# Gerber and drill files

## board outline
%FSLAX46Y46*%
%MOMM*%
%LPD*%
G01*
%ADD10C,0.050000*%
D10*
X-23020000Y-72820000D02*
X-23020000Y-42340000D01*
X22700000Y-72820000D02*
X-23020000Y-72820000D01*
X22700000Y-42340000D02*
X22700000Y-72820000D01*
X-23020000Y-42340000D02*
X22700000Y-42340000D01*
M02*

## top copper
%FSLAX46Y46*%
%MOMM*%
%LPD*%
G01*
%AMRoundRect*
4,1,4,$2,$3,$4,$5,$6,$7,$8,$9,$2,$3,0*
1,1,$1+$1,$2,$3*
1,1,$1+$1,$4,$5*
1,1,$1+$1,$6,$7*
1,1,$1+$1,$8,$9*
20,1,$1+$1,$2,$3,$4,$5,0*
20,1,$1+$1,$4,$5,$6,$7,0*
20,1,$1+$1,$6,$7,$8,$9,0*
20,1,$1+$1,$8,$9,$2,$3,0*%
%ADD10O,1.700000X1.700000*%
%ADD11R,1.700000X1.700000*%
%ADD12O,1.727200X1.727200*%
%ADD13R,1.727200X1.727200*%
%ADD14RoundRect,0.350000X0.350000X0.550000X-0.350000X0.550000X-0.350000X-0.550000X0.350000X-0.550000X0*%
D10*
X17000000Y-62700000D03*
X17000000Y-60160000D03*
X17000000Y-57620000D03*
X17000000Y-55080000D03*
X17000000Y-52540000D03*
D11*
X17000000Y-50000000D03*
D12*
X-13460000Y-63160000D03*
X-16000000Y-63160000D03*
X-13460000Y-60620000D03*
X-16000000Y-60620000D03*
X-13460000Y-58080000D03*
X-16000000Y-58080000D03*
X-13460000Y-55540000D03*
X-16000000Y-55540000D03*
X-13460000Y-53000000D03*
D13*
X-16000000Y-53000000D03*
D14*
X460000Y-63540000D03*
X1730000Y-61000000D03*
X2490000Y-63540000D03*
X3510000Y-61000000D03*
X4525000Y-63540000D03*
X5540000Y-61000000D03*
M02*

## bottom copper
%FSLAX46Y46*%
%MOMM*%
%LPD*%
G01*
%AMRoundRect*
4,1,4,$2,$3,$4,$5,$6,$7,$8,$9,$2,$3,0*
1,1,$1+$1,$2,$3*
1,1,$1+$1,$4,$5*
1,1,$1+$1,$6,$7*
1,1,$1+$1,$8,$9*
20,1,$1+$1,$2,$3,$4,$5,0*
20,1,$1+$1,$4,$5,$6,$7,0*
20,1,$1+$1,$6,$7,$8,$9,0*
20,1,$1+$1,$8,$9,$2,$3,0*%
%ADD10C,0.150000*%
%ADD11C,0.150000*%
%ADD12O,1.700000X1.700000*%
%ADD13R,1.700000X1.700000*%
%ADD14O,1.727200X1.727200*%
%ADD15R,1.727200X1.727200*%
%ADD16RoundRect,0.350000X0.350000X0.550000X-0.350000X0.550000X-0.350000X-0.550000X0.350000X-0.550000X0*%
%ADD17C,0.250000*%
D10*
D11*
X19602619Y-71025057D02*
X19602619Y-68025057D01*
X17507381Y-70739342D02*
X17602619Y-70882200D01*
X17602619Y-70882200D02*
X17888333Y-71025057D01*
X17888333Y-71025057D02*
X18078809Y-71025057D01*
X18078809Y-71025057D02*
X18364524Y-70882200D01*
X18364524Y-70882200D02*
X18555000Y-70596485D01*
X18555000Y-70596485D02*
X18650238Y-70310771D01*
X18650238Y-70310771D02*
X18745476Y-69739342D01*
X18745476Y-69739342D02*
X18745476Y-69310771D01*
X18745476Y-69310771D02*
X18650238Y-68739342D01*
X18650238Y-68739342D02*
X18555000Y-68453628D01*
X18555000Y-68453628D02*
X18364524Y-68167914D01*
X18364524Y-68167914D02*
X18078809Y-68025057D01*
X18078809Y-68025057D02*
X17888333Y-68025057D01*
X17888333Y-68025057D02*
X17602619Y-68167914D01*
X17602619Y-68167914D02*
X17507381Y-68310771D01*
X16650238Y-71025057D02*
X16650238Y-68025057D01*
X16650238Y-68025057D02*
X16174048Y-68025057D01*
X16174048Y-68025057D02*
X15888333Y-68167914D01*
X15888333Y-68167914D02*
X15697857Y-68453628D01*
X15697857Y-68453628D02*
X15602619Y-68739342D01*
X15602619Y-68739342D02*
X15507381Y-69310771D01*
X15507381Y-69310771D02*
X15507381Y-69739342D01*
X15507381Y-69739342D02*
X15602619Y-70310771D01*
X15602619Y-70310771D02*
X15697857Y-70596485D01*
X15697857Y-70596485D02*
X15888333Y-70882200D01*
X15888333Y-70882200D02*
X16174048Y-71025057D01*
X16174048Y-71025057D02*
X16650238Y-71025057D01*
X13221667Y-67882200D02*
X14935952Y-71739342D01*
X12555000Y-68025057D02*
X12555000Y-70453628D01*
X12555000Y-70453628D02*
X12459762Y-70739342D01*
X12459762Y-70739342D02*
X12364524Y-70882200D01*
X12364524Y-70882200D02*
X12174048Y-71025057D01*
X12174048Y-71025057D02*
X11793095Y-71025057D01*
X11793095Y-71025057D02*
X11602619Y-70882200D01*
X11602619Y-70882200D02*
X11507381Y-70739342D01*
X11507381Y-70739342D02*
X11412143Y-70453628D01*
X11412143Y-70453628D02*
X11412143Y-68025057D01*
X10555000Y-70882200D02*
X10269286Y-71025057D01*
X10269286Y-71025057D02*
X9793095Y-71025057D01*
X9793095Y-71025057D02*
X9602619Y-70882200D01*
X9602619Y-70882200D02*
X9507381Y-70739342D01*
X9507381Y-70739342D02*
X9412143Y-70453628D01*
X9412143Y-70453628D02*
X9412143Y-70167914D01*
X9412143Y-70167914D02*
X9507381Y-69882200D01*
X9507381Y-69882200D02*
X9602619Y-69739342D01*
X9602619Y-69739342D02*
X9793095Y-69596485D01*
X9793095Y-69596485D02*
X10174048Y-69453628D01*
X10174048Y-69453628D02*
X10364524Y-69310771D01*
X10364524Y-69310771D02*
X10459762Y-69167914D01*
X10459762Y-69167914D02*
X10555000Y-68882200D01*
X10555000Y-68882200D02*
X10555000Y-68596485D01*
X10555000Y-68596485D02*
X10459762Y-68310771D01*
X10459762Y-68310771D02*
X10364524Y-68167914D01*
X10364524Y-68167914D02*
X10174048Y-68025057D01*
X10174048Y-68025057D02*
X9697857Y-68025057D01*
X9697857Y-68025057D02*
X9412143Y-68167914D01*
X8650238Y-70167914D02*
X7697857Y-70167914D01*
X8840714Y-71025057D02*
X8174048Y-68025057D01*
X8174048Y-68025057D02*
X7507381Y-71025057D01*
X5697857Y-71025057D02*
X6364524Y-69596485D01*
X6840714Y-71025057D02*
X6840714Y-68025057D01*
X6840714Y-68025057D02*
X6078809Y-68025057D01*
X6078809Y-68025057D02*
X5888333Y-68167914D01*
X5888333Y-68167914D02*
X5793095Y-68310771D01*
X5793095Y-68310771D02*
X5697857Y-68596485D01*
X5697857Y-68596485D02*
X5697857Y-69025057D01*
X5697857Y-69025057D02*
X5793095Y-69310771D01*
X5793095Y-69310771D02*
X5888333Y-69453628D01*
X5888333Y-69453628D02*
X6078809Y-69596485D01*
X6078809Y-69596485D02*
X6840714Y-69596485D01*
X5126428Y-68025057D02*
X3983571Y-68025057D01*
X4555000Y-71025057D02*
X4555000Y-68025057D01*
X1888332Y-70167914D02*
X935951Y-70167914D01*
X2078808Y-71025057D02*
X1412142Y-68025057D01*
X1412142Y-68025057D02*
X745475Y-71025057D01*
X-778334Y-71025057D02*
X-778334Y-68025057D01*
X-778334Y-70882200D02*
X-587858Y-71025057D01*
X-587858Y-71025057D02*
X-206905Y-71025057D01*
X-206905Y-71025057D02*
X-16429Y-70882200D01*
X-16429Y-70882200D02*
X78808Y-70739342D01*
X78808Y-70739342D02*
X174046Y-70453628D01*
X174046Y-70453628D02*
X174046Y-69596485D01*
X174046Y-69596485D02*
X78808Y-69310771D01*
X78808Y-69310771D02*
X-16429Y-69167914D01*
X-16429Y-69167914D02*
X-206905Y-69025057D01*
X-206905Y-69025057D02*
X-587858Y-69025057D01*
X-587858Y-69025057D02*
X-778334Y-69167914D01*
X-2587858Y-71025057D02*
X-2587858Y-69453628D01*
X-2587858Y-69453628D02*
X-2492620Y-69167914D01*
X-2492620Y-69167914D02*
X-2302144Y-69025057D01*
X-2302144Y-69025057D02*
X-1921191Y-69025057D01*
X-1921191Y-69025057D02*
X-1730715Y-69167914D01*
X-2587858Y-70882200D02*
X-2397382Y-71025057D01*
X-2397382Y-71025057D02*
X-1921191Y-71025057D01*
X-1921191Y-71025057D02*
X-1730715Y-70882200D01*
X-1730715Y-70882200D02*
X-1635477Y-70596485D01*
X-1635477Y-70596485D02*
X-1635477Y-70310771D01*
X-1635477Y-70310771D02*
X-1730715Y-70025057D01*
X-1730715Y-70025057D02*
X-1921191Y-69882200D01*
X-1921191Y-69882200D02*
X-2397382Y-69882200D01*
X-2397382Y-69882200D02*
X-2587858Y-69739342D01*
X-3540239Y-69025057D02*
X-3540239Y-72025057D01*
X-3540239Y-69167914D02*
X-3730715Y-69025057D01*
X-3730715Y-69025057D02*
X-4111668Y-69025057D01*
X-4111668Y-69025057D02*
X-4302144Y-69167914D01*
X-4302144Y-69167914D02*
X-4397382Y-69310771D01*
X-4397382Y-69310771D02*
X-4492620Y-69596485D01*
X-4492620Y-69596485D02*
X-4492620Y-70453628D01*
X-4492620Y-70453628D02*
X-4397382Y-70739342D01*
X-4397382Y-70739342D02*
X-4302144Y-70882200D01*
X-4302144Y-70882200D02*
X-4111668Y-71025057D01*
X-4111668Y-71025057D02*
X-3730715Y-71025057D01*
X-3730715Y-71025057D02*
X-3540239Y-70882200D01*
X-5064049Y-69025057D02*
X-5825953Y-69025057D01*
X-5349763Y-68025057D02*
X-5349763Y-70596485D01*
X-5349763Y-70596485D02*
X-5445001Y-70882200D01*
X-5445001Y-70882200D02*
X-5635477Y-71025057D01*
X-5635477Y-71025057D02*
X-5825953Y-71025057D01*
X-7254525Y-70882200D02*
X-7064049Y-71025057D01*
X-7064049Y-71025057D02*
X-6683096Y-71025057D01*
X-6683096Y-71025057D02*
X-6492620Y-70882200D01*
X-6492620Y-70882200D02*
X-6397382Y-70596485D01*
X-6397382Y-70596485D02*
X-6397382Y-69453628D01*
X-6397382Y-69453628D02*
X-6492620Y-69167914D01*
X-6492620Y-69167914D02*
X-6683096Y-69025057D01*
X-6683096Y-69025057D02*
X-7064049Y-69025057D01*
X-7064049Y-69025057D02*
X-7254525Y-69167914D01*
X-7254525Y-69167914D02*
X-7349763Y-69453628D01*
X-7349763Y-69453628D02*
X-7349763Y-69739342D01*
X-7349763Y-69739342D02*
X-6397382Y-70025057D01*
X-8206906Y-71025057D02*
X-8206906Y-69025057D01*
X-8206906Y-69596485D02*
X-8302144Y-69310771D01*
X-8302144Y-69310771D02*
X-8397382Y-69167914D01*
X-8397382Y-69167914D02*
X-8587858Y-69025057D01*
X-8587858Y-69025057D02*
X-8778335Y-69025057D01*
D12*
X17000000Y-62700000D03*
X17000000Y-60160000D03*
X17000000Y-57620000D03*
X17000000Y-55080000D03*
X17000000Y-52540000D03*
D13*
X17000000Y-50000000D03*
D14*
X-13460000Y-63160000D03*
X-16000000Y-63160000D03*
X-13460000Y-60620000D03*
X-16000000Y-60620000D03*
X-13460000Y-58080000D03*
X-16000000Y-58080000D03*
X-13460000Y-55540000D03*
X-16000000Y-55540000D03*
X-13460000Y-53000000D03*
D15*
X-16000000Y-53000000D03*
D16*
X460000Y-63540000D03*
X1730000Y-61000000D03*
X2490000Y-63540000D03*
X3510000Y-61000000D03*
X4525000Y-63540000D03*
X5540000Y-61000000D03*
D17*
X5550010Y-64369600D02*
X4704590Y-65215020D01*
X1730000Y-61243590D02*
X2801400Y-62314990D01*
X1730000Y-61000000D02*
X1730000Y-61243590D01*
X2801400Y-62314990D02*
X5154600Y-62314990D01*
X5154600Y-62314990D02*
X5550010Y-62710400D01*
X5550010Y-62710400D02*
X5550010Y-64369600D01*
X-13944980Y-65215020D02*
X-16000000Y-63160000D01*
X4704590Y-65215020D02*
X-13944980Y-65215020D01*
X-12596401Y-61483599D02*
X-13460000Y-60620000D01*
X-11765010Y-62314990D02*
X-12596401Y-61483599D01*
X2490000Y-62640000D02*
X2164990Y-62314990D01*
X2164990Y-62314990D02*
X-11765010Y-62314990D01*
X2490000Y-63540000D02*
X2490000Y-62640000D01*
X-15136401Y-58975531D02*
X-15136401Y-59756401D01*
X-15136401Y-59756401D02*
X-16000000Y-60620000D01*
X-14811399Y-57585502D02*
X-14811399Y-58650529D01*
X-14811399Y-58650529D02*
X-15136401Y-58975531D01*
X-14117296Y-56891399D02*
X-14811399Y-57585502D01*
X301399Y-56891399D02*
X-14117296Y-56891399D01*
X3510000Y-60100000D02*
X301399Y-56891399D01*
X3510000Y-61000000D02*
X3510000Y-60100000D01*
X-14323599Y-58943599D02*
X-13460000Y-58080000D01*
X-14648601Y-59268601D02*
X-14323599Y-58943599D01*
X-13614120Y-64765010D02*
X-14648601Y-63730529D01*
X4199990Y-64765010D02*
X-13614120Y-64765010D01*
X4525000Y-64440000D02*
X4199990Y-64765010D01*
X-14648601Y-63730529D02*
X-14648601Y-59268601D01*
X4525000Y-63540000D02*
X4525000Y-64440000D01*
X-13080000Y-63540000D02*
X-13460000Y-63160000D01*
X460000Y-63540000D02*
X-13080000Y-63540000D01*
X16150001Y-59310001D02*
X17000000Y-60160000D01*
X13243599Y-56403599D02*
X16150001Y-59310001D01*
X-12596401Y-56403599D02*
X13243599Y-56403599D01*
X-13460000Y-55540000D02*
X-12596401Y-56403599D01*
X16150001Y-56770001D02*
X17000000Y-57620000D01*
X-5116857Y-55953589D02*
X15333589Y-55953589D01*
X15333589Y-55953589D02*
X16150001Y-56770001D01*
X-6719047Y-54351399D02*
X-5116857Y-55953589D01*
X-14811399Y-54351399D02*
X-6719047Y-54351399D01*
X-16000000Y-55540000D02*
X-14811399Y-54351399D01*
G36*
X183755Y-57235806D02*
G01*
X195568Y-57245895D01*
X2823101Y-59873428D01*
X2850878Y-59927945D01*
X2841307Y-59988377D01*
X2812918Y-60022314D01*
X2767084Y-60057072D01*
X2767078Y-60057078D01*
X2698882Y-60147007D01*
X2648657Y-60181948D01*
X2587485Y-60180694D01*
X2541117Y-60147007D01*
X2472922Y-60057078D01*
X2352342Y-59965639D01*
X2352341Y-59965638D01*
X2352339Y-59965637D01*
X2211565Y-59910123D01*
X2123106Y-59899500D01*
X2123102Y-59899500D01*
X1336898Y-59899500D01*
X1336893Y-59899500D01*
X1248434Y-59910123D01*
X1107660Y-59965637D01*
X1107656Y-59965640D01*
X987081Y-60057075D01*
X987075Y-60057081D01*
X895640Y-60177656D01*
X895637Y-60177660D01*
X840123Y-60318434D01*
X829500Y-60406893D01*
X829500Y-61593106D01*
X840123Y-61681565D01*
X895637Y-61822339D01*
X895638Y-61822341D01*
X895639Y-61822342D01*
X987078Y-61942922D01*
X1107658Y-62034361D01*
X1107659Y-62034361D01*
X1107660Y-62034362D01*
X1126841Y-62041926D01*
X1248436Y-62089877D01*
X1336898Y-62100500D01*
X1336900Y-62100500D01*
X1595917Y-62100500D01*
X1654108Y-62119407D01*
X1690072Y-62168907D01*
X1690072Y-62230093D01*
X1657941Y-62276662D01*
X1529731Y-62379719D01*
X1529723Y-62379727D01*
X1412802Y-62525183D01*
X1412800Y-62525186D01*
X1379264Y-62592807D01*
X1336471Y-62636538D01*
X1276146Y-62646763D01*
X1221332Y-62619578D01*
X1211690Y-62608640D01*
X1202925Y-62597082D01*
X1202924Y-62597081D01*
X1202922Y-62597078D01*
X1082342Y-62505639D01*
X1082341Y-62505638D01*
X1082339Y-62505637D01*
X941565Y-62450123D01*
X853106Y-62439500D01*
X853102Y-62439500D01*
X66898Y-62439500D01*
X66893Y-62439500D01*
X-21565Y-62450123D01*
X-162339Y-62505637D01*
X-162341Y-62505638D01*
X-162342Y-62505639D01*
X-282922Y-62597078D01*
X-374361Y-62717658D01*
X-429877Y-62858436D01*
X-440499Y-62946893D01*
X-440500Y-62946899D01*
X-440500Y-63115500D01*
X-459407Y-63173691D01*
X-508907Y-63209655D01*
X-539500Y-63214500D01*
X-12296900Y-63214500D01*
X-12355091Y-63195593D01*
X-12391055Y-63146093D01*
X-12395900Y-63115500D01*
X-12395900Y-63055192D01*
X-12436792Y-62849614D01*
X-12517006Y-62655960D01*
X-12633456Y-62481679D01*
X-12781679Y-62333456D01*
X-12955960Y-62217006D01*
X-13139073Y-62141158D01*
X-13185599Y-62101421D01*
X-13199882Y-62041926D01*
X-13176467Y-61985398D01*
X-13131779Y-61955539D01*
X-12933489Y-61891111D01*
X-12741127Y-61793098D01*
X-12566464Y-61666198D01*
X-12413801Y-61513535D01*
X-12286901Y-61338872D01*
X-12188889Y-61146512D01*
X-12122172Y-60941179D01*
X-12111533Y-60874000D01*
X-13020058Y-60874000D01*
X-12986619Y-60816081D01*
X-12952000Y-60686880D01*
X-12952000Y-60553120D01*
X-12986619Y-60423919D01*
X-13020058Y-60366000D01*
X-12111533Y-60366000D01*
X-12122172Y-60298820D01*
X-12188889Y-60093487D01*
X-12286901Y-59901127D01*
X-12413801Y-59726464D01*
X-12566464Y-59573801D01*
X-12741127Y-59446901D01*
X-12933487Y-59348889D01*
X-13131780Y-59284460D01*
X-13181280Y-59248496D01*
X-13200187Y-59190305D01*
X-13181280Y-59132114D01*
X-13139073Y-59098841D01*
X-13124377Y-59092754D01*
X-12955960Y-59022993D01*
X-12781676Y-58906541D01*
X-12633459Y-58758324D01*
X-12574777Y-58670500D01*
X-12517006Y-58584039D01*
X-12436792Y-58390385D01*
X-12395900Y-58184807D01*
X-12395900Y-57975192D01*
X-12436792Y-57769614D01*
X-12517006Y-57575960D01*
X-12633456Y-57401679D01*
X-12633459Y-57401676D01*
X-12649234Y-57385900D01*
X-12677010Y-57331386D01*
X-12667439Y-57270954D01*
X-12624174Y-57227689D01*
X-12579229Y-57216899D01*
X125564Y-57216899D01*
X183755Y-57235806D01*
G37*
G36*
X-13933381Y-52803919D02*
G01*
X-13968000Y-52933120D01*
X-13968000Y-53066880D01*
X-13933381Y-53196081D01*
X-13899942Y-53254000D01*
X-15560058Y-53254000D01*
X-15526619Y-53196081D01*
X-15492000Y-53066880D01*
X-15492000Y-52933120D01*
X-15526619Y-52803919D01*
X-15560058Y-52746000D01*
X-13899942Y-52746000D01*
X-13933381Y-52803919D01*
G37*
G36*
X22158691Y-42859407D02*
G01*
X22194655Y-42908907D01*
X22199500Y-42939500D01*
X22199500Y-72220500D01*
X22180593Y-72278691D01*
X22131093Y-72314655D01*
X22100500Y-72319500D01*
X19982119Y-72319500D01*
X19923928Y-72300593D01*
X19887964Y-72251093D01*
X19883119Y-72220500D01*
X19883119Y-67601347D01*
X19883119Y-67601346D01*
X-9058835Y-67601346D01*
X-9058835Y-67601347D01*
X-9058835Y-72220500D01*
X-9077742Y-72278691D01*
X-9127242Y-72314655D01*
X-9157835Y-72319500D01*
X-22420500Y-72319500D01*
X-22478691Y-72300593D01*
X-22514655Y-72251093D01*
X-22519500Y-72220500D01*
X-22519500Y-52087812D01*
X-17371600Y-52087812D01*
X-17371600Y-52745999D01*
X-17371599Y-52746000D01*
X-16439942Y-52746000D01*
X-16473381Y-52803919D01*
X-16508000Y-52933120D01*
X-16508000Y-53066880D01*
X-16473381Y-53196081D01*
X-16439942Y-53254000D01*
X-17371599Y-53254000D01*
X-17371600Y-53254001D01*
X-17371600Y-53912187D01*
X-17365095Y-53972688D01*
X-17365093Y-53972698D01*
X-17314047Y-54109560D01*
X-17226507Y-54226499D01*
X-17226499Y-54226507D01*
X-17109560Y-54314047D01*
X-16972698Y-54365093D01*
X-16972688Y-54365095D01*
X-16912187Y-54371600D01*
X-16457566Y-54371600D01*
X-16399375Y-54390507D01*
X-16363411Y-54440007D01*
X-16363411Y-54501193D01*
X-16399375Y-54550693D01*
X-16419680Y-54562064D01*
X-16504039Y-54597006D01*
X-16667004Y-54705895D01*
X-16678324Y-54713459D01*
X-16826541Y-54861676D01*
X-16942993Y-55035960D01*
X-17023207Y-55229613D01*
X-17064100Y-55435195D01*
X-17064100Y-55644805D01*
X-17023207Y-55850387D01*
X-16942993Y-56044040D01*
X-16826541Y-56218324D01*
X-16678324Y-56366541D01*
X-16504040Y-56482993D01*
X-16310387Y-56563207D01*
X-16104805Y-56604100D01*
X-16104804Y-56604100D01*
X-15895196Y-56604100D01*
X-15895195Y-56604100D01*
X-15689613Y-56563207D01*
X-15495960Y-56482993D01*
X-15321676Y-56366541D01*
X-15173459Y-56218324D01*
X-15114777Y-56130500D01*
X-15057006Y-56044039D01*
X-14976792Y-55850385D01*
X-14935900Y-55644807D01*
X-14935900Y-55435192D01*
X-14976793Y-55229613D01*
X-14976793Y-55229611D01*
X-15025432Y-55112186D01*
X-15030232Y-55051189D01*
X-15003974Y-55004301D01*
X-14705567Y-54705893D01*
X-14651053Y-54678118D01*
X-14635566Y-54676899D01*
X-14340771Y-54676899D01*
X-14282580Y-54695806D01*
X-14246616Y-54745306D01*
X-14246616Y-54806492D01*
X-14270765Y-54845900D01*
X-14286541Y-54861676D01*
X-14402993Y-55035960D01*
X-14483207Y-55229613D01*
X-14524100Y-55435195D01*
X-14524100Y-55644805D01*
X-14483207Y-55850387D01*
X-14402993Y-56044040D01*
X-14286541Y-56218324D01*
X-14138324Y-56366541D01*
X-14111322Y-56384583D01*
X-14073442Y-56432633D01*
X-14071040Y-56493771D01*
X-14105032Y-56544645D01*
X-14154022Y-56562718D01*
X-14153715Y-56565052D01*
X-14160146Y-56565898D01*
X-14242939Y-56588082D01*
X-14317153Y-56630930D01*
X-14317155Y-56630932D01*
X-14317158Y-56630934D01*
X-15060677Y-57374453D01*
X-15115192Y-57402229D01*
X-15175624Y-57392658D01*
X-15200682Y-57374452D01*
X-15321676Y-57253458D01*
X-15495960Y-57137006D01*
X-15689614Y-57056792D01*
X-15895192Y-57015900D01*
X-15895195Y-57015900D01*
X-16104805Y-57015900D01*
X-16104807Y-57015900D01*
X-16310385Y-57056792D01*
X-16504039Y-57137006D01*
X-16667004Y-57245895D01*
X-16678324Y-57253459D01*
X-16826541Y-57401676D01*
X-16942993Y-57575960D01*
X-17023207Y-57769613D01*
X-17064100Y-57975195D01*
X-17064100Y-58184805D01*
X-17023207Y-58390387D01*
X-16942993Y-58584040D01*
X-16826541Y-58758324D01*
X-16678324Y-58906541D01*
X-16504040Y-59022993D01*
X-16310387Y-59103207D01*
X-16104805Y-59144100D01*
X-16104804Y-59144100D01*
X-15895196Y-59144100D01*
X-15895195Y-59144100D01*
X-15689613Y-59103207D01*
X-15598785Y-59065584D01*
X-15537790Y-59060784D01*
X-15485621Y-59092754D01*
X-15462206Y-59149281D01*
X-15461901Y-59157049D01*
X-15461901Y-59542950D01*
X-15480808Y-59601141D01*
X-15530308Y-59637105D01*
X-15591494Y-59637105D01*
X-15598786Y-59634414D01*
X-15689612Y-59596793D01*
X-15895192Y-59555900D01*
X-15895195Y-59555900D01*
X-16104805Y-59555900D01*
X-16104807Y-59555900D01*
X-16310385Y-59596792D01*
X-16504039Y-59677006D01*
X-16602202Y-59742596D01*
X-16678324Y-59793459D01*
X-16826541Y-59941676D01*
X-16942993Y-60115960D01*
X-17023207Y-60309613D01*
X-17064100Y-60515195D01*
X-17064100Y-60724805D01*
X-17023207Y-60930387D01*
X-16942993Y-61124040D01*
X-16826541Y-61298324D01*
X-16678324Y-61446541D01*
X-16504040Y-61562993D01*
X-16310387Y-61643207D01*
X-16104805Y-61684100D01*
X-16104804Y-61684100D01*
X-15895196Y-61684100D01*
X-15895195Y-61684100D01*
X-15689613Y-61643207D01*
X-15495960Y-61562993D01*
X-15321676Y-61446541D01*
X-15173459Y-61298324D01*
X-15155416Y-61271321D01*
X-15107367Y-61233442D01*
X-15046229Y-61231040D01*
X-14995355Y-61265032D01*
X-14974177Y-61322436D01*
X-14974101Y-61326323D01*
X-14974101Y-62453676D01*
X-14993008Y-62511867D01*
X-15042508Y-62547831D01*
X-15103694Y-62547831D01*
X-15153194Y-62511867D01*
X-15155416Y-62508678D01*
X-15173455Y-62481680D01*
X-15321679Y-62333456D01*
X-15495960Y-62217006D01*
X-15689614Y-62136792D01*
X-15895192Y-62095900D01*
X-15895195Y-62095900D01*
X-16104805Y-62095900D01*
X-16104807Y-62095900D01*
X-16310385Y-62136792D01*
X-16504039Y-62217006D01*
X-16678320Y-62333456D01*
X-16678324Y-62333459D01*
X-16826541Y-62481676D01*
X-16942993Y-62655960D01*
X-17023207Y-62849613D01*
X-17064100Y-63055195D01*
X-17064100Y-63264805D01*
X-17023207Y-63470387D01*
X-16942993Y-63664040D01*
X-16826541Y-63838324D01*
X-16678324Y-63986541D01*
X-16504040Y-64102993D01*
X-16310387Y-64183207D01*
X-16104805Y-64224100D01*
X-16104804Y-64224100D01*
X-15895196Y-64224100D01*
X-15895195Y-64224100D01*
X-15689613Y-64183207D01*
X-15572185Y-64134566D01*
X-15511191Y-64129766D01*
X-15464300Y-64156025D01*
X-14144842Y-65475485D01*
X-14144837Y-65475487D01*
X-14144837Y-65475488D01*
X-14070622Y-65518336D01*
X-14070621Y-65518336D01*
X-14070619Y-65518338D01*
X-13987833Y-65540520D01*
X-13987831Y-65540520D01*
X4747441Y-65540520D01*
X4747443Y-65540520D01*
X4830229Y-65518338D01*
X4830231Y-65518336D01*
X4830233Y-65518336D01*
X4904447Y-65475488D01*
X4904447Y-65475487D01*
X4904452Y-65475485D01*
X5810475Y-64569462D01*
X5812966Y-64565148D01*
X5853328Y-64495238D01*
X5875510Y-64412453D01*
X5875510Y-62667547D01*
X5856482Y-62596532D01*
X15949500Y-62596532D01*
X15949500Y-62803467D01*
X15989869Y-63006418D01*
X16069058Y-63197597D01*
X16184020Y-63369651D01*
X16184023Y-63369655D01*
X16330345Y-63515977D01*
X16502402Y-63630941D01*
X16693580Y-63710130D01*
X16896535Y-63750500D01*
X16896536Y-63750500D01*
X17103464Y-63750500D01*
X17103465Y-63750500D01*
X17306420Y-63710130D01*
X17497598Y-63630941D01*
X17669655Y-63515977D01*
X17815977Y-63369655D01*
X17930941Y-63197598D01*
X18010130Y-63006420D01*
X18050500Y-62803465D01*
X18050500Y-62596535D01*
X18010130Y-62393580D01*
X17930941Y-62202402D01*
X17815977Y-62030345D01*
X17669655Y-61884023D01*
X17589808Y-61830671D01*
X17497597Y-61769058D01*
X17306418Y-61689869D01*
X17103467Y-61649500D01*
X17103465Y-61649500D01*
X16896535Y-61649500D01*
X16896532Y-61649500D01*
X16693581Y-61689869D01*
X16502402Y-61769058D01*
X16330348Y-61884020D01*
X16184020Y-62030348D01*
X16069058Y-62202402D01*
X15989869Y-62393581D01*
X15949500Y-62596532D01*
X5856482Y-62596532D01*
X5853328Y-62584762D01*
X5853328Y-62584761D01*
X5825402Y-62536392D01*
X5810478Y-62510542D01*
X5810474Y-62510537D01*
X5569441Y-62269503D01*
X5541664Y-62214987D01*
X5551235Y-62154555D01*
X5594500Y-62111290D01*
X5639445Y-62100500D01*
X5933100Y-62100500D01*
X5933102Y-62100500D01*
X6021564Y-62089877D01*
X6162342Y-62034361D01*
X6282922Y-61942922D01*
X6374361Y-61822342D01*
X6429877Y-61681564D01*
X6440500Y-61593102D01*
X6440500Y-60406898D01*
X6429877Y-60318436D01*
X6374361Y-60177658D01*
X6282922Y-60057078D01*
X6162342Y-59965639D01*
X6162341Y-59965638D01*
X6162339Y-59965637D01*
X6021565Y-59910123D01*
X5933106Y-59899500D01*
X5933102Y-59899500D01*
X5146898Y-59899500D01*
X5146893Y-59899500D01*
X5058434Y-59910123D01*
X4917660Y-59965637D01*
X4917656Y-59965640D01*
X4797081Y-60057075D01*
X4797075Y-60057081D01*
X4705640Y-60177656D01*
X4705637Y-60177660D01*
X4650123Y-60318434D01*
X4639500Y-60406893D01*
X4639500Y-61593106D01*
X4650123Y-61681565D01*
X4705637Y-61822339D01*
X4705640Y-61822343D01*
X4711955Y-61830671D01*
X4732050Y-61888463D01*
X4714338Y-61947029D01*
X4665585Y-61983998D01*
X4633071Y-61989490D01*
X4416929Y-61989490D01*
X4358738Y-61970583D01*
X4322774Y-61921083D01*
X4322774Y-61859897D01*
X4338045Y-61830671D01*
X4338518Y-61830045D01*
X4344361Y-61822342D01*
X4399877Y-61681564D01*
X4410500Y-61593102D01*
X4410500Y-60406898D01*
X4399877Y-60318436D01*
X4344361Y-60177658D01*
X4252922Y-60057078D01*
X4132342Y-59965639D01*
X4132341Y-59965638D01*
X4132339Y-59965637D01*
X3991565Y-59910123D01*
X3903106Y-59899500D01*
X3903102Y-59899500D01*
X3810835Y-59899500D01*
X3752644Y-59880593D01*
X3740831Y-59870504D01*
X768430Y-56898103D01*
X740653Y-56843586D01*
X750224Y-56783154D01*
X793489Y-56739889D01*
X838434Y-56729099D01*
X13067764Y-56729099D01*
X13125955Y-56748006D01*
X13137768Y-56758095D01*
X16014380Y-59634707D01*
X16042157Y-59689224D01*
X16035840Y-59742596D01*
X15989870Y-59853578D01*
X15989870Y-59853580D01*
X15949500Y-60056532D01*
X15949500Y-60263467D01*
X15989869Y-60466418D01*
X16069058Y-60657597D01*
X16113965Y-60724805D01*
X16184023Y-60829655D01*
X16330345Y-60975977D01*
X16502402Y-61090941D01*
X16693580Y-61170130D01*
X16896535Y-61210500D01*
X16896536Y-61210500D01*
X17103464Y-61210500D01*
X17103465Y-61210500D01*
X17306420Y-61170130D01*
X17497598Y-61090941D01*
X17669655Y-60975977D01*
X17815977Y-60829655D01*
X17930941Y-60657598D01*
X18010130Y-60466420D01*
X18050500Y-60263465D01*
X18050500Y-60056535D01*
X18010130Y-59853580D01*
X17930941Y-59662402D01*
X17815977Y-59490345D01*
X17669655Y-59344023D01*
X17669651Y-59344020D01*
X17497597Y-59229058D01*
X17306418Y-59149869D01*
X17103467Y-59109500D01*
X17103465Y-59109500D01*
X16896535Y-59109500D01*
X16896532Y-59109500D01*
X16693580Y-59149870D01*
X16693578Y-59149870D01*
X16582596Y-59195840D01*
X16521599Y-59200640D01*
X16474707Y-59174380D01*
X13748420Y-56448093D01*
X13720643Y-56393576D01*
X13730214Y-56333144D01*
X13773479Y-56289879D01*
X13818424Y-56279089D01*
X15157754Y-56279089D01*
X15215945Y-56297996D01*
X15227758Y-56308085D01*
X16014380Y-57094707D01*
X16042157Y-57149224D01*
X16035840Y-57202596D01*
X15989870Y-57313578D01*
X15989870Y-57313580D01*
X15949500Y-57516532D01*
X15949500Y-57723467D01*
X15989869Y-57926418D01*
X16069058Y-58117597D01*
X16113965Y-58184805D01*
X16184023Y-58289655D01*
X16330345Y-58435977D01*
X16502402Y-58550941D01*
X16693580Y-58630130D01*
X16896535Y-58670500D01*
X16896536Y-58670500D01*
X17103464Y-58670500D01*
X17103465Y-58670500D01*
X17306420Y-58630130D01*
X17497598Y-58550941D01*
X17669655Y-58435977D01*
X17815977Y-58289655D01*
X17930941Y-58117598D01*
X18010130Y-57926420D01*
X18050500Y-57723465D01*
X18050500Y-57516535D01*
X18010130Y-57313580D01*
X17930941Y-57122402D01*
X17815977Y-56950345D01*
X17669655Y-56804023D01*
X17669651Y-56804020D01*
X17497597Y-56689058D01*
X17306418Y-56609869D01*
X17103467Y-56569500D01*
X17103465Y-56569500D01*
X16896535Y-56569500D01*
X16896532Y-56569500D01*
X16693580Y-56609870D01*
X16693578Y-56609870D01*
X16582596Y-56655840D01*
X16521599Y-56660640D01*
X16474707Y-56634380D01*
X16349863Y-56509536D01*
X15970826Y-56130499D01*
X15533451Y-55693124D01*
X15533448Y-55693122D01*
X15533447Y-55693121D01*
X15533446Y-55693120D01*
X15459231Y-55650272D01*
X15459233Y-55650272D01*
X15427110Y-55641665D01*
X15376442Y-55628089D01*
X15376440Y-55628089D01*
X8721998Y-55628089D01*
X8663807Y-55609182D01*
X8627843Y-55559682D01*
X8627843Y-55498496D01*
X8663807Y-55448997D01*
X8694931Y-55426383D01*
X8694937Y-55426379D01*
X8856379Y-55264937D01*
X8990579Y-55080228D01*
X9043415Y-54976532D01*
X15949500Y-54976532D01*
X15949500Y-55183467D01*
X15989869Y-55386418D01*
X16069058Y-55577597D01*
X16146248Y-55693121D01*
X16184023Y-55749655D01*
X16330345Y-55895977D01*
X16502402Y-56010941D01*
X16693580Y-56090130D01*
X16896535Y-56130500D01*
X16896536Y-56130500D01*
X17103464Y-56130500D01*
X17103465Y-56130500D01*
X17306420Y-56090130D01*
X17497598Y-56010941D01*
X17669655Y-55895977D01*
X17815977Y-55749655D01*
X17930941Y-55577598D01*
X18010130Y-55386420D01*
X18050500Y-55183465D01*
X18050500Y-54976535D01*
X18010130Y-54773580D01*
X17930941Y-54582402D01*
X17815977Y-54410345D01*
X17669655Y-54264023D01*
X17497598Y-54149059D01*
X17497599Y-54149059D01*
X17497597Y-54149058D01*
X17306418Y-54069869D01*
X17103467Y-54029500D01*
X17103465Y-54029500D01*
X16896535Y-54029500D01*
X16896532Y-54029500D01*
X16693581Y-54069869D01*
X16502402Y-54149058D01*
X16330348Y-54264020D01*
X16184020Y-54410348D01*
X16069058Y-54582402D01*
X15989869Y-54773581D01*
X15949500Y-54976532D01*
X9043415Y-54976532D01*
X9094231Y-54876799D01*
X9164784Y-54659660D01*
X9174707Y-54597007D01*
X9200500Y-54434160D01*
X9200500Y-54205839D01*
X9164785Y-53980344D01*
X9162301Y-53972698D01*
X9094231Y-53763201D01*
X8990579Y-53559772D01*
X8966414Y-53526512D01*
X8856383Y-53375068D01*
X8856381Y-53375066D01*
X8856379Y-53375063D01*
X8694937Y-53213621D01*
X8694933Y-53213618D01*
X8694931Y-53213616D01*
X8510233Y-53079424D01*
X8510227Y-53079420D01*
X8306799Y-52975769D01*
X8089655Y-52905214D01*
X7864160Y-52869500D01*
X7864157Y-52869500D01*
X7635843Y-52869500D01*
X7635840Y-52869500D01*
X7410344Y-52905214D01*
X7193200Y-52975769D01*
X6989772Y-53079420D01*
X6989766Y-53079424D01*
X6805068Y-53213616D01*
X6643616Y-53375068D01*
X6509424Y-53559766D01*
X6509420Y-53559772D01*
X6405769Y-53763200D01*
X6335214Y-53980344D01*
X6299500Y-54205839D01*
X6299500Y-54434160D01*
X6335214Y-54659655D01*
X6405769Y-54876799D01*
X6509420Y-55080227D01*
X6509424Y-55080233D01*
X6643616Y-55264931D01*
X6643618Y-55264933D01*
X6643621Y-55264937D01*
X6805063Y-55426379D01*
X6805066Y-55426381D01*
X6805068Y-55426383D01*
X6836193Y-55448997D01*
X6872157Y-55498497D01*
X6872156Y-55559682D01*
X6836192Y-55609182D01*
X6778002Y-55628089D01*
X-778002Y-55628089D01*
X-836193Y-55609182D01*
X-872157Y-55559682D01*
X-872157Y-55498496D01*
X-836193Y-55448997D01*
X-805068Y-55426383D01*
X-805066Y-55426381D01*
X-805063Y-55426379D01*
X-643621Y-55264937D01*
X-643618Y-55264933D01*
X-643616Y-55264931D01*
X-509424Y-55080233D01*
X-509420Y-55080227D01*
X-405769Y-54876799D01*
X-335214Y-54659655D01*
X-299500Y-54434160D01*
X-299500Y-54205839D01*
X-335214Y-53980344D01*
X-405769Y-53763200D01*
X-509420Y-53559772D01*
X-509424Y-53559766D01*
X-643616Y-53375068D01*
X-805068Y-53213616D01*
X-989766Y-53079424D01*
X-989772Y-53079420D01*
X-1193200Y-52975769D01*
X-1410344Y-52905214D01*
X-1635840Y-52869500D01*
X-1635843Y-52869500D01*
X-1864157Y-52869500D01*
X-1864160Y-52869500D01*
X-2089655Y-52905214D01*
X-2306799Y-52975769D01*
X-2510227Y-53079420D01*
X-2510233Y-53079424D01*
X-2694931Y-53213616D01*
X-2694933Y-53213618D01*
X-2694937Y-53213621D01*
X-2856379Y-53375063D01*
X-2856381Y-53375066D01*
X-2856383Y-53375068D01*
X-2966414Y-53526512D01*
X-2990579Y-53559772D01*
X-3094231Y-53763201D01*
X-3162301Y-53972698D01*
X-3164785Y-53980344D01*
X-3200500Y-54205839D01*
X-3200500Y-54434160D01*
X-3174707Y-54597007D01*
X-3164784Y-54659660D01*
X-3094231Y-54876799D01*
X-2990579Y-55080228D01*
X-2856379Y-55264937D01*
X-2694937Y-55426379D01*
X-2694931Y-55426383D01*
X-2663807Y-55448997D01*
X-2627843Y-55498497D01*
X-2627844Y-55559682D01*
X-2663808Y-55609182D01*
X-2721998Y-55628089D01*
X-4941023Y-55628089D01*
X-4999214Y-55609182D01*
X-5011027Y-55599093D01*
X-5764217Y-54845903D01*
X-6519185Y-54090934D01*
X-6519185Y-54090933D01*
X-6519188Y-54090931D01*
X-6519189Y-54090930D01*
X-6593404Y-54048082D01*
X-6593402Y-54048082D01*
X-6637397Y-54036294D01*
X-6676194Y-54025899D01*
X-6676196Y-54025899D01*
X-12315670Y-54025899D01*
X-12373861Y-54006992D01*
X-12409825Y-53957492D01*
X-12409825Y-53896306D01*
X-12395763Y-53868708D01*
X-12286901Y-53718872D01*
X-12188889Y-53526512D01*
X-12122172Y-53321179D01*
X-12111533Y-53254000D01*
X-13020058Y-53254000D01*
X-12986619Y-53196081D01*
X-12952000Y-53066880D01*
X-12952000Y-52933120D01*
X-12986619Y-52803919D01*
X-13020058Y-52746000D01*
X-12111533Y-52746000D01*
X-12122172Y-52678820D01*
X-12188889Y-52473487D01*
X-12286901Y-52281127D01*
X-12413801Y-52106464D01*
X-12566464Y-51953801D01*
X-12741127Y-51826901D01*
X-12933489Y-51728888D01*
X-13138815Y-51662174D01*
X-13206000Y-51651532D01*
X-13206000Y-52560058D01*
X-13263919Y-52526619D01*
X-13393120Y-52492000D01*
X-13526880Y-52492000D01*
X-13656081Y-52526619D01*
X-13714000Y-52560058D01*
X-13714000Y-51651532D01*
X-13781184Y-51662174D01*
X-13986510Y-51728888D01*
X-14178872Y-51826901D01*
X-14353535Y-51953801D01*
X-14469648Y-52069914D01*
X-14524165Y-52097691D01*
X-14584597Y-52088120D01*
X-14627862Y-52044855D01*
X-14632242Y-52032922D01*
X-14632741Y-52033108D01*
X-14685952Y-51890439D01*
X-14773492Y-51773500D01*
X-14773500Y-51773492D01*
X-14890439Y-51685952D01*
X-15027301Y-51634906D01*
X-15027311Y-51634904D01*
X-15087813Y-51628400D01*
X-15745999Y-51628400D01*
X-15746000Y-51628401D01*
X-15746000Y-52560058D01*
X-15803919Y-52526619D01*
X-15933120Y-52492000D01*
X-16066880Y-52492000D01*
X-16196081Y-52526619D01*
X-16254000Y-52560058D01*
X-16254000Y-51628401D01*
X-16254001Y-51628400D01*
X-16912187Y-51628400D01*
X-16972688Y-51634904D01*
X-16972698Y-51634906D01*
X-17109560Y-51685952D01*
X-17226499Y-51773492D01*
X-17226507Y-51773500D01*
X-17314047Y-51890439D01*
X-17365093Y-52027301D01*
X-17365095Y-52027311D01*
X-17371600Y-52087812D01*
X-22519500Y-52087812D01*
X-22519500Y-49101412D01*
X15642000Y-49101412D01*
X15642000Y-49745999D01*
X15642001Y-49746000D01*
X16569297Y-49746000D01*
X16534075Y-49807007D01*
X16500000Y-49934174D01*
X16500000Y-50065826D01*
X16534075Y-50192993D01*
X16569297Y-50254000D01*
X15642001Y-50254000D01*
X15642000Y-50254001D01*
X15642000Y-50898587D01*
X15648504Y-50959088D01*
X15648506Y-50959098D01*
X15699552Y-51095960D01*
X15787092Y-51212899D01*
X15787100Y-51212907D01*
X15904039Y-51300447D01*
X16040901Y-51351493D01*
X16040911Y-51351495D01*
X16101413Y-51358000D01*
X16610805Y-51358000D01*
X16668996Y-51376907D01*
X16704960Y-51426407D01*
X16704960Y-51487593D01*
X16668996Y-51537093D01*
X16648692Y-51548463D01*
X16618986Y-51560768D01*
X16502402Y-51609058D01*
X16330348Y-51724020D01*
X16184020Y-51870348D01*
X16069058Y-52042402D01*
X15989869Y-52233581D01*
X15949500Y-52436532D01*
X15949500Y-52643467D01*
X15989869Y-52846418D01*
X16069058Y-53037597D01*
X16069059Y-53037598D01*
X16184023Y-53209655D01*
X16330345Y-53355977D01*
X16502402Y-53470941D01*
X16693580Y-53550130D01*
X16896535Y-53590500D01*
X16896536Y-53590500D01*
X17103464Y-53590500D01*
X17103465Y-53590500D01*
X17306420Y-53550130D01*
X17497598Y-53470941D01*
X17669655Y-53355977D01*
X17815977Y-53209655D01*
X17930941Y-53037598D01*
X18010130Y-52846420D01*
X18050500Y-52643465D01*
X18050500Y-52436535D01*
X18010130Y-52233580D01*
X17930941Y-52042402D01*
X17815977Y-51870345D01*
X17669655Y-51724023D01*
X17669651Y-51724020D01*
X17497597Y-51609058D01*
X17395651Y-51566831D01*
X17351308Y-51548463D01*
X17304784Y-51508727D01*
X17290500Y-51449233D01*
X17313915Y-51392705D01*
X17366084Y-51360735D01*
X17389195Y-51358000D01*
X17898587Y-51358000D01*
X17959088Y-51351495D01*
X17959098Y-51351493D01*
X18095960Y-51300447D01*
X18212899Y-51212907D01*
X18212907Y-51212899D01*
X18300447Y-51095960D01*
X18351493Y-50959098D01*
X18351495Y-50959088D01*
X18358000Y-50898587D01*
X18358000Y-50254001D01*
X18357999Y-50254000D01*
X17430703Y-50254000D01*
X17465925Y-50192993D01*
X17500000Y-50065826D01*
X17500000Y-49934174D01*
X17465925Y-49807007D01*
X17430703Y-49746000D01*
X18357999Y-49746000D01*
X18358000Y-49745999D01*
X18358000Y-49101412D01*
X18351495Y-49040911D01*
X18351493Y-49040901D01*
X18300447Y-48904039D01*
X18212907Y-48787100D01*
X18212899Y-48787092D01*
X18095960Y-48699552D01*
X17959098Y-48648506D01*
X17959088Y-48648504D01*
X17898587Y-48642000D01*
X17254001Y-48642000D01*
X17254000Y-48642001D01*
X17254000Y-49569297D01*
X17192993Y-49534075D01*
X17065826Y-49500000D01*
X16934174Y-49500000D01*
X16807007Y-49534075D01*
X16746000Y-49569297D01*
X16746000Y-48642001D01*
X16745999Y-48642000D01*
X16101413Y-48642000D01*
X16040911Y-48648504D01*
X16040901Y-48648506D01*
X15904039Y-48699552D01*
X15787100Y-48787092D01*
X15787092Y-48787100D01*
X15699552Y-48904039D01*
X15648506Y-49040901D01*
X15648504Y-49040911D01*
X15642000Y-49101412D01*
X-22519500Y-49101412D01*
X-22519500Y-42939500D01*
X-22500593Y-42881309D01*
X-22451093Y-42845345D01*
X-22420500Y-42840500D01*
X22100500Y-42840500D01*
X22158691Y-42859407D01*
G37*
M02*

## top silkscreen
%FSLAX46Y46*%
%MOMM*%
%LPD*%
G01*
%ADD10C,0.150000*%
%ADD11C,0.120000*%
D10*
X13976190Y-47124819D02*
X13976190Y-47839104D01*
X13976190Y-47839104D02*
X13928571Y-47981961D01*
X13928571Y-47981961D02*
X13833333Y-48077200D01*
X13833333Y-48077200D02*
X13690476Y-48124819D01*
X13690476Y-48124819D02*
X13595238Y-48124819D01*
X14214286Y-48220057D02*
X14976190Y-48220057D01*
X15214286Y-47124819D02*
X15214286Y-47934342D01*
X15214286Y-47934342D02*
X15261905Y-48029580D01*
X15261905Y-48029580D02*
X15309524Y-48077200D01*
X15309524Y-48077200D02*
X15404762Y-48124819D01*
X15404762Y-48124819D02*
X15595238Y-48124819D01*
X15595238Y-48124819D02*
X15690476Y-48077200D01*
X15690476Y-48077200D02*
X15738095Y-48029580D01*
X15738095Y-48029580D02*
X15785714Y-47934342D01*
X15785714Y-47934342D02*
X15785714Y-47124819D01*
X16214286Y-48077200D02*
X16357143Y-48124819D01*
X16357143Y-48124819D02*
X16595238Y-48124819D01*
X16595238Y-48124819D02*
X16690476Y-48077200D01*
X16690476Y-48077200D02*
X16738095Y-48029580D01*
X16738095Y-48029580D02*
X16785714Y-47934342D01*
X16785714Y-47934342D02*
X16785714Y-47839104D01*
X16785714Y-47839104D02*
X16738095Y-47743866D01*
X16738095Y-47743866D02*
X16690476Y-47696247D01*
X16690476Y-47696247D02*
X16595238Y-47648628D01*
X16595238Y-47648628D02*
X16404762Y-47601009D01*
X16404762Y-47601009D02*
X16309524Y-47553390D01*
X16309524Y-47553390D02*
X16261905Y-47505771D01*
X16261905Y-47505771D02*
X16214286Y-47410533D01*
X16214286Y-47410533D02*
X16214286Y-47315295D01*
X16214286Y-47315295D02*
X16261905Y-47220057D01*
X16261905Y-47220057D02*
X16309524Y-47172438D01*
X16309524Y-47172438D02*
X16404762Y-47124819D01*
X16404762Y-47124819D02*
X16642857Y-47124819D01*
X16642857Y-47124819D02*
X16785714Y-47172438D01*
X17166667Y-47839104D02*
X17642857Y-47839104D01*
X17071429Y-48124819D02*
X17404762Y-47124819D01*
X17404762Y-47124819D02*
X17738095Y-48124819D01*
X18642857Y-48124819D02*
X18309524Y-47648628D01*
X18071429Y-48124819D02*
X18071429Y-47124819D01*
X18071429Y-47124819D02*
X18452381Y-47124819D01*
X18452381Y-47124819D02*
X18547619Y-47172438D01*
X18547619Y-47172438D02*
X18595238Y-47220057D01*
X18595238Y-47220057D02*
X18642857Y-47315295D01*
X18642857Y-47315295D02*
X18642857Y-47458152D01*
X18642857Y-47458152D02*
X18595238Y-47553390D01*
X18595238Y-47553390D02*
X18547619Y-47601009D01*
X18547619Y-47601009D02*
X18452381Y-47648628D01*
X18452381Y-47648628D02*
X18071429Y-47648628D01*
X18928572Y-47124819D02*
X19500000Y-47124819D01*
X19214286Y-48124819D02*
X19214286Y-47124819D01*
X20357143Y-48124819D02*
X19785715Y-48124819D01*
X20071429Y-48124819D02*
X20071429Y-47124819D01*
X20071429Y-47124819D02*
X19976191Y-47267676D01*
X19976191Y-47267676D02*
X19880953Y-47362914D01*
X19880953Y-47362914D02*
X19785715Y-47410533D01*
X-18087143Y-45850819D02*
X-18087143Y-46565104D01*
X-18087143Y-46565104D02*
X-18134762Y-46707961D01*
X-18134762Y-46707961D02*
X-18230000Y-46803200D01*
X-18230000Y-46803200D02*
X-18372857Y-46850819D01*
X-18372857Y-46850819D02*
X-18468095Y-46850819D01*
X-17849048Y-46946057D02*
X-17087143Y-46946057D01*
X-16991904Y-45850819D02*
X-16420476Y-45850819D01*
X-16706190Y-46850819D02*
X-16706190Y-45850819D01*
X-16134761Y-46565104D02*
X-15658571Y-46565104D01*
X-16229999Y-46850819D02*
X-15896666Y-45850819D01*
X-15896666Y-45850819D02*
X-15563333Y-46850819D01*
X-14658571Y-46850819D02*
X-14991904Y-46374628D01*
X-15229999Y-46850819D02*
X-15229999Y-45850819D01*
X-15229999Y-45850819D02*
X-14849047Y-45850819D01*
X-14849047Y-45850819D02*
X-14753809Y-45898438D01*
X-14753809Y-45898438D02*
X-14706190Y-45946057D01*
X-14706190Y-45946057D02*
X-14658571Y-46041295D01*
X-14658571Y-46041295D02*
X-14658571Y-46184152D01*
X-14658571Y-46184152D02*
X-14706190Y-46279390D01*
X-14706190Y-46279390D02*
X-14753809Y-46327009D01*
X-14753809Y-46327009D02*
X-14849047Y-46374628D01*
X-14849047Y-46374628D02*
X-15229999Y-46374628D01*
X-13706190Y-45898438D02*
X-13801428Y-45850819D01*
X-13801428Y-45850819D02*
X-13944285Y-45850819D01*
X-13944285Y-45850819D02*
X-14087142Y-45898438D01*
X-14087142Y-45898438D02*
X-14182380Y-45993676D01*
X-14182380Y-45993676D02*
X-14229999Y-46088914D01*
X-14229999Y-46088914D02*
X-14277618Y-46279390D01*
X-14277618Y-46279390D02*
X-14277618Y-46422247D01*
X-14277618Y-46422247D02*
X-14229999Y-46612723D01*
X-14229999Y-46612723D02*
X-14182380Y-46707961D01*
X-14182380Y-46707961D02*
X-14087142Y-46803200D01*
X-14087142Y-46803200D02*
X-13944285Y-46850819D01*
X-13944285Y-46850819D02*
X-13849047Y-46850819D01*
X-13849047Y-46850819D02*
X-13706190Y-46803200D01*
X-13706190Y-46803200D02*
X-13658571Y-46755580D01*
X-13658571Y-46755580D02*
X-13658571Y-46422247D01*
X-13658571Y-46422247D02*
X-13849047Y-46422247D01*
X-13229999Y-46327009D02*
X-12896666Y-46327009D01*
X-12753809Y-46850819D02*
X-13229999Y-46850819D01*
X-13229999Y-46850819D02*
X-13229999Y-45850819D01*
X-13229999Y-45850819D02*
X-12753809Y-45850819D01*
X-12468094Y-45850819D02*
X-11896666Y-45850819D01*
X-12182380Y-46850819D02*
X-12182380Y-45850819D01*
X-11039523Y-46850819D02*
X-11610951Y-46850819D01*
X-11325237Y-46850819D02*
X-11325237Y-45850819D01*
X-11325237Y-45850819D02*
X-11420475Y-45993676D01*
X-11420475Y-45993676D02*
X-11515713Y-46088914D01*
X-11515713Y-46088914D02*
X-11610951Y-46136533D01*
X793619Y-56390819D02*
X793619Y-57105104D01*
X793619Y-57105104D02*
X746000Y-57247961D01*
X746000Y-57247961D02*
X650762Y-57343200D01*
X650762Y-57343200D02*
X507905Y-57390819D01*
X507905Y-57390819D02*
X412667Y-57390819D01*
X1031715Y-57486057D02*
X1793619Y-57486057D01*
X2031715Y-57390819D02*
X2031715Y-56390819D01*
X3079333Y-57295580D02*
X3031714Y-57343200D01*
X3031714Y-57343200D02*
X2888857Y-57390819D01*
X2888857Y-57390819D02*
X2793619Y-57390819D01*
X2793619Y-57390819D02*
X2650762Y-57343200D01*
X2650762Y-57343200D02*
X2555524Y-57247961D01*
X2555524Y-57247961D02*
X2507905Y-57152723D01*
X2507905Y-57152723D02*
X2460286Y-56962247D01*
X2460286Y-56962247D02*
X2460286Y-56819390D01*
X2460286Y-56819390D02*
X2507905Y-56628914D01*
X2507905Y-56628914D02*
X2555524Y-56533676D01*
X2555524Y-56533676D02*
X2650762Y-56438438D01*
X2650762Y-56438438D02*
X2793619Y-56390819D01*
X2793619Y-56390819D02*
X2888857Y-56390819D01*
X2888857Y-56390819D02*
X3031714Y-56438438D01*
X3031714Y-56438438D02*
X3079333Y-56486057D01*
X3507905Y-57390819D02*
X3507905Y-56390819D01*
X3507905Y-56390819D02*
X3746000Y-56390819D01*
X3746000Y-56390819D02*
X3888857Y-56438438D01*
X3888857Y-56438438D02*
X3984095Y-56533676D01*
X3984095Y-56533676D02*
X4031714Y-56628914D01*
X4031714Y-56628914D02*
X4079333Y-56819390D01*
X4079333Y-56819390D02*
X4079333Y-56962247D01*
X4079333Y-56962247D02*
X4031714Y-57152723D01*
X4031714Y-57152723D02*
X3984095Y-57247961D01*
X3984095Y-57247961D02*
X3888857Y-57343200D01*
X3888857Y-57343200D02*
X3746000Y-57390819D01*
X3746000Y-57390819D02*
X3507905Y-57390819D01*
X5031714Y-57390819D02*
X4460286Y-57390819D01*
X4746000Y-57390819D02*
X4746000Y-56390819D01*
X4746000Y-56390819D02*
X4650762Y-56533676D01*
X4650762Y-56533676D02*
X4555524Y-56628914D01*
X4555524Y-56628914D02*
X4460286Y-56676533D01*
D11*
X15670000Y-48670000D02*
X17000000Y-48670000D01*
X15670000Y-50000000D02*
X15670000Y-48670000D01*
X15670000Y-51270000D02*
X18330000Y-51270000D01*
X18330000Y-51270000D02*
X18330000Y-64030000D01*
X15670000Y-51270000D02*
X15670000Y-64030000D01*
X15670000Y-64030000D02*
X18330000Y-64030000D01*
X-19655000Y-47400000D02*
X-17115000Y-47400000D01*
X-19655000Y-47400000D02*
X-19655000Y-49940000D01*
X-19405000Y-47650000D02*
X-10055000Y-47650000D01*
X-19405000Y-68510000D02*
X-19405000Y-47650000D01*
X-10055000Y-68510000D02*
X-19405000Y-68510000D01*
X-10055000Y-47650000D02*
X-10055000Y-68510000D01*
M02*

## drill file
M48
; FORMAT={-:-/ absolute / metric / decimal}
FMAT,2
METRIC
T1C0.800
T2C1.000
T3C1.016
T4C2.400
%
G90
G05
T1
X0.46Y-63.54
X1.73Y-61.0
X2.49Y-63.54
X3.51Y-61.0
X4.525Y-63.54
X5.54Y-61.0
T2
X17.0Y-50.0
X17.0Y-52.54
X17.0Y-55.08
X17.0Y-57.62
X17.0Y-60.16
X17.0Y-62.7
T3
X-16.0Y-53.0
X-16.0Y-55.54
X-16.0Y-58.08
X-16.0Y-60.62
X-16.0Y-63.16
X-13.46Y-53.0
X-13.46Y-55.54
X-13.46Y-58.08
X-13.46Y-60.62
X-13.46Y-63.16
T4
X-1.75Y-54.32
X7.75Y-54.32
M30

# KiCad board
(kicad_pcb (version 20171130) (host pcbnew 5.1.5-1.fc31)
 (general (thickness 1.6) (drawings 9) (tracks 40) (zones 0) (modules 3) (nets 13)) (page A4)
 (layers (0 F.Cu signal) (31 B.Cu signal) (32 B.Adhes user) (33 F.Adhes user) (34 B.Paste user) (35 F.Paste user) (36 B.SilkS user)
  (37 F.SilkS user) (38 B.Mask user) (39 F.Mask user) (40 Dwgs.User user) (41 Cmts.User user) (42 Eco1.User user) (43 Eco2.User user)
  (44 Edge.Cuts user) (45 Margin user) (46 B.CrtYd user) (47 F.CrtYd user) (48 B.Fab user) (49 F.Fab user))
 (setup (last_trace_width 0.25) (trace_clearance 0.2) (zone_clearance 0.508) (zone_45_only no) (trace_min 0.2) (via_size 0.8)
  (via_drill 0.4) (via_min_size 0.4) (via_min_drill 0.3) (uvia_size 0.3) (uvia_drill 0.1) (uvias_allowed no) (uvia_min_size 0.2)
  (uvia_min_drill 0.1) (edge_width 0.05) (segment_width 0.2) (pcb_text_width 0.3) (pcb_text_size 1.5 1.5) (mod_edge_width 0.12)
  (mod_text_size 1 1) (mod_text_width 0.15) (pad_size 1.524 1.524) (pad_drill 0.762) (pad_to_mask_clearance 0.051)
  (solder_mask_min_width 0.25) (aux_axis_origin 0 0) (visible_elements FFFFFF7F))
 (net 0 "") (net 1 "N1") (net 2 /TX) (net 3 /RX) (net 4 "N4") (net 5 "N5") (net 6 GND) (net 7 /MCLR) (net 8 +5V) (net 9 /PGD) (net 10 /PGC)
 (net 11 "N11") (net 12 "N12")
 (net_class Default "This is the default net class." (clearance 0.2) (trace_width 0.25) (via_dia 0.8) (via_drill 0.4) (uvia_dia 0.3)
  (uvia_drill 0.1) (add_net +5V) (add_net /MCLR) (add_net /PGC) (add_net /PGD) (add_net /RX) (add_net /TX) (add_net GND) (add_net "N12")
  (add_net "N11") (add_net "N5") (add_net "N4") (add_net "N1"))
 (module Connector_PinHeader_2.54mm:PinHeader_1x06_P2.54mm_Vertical (layer F.Cu) (at 17 50)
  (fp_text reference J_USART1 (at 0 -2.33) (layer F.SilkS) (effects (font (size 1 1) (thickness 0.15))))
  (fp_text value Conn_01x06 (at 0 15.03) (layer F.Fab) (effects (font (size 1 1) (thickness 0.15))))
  (fp_line (start -1.33 -1.33) (end 0 -1.33) (layer F.SilkS) (width 0.12))
  (fp_line (start -1.33 0) (end -1.33 -1.33) (layer F.SilkS) (width 0.12))
  (fp_line (start -1.33 1.27) (end 1.33 1.27) (layer F.SilkS) (width 0.12))
  (fp_line (start 1.33 1.27) (end 1.33 14.03) (layer F.SilkS) (width 0.12))
  (fp_line (start -1.33 1.27) (end -1.33 14.03) (layer F.SilkS) (width 0.12))
  (fp_line (start -1.33 14.03) (end 1.33 14.03) (layer F.SilkS) (width 0.12))
  (pad 6 thru_hole oval (at 0 12.7) (size 1.7 1.7) (drill 1) (layers *.Cu *.Mask) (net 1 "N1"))
  (pad 5 thru_hole oval (at 0 10.16) (size 1.7 1.7) (drill 1) (layers *.Cu *.Mask) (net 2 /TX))
  (pad 4 thru_hole oval (at 0 7.62) (size 1.7 1.7) (drill 1) (layers *.Cu *.Mask) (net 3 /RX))
  (pad 3 thru_hole oval (at 0 5.08) (size 1.7 1.7) (drill 1) (layers *.Cu *.Mask) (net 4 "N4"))
  (pad 2 thru_hole oval (at 0 2.54) (size 1.7 1.7) (drill 1) (layers *.Cu *.Mask) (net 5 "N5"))
  (pad 1 thru_hole rect (at 0 0) (size 1.7 1.7) (drill 1) (layers *.Cu *.Mask) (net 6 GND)))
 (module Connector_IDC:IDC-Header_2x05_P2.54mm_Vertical (layer F.Cu) (at -16 53)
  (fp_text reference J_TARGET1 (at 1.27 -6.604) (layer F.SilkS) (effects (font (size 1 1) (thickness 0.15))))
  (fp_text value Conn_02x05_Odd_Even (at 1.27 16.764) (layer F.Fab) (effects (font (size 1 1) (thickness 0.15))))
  (fp_line (start -3.655 -5.6) (end -1.115 -5.6) (layer F.SilkS) (width 0.12))
  (fp_line (start -3.655 -5.6) (end -3.655 -3.06) (layer F.SilkS) (width 0.12))
  (fp_line (start -3.405 -5.35) (end 5.945 -5.35) (layer F.SilkS) (width 0.12))
  (fp_line (start -3.405 15.51) (end -3.405 -5.35) (layer F.SilkS) (width 0.12))
  (fp_line (start 5.945 15.51) (end -3.405 15.51) (layer F.SilkS) (width 0.12))
  (fp_line (start 5.945 -5.35) (end 5.945 15.51) (layer F.SilkS) (width 0.12))
  (pad 10 thru_hole oval (at 2.54 10.16) (size 1.7272 1.7272) (drill 1.016) (layers *.Cu *.Mask) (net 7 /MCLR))
  (pad 9 thru_hole oval (at 0 10.16) (size 1.7272 1.7272) (drill 1.016) (layers *.Cu *.Mask) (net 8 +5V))
  (pad 8 thru_hole oval (at 2.54 7.62) (size 1.7272 1.7272) (drill 1.016) (layers *.Cu *.Mask) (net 6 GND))
  (pad 7 thru_hole oval (at 0 7.62) (size 1.7272 1.7272) (drill 1.016) (layers *.Cu *.Mask) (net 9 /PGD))
  (pad 6 thru_hole oval (at 2.54 5.08) (size 1.7272 1.7272) (drill 1.016) (layers *.Cu *.Mask) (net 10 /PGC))
  (pad 5 thru_hole oval (at 0 5.08) (size 1.7272 1.7272) (drill 1.016) (layers *.Cu *.Mask) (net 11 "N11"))
  (pad 4 thru_hole oval (at 2.54 2.54) (size 1.7272 1.7272) (drill 1.016) (layers *.Cu *.Mask) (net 2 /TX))
  (pad 3 thru_hole oval (at 0 2.54) (size 1.7272 1.7272) (drill 1.016) (layers *.Cu *.Mask) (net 3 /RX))
  (pad 2 thru_hole oval (at 2.54 0) (size 1.7272 1.7272) (drill 1.016) (layers *.Cu *.Mask) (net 6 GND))
  (pad 1 thru_hole rect (at 0 0) (size 1.7272 1.7272) (drill 1.016) (layers *.Cu *.Mask) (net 6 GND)))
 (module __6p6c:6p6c (layer F.Cu) (at 3 61 180)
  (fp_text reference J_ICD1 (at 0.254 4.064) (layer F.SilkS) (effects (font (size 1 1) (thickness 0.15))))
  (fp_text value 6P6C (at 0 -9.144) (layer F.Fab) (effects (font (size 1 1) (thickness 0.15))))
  (pad "" np_thru_hole circle (at 4.75 6.68 180) (size 2.4 2.4) (drill 2.4) (layers *.Cu *.Mask))
  (pad "" np_thru_hole circle (at -4.75 6.68 180) (size 2.4 2.4) (drill 2.4) (layers *.Cu *.Mask))
  (pad 6 thru_hole roundrect (at 2.54 -2.54 180) (size 1.4 1.8) (drill 0.8) (layers *.Cu *.Mask) (roundrect_rratio 0.25) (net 7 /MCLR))
  (pad 5 thru_hole roundrect (at 1.27 0 180) (size 1.4 1.8) (drill 0.8) (layers *.Cu *.Mask) (roundrect_rratio 0.25) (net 8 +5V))
  (pad 4 thru_hole roundrect (at 0.51 -2.54 180) (size 1.4 1.8) (drill 0.8) (layers *.Cu *.Mask) (roundrect_rratio 0.25) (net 6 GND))
  (pad 3 thru_hole roundrect (at -0.51 0 180) (size 1.4 1.8) (drill 0.8) (layers *.Cu *.Mask) (roundrect_rratio 0.25) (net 9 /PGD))
  (pad 2 thru_hole roundrect (at -1.525 -2.54 180) (size 1.4 1.8) (drill 0.8) (layers *.Cu *.Mask) (roundrect_rratio 0.25) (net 10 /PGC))
  (pad 1 thru_hole roundrect (at -2.54 0 180) (size 1.4 1.8) (drill 0.8) (layers *.Cu *.Mask) (roundrect_rratio 0.25) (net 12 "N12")))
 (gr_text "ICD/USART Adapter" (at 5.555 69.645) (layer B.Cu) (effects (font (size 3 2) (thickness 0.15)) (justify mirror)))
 (gr_line (start -23.02 72.82) (end -23.02 42.34) (layer Edge.Cuts) (width 0.05))
 (gr_line (start 22.7 72.82) (end -23.02 72.82) (layer Edge.Cuts) (width 0.05))
 (gr_line (start 22.7 42.34) (end 22.7 72.82) (layer Edge.Cuts) (width 0.05))
 (gr_line (start -23.02 42.34) (end 22.7 42.34) (layer Edge.Cuts) (width 0.05))
 (segment (start 5.55001 64.3696) (end 4.70459 65.21502) (width 0.25) (layer B.Cu) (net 8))
 (segment (start 1.73 61.24359) (end 2.8014 62.31499) (width 0.25) (layer B.Cu) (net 8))
 (segment (start 1.73 61) (end 1.73 61.24359) (width 0.25) (layer B.Cu) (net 8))
 (segment (start 2.8014 62.31499) (end 5.1546 62.31499) (width 0.25) (layer B.Cu) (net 8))
 (segment (start 5.1546 62.31499) (end 5.55001 62.7104) (width 0.25) (layer B.Cu) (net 8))
 (segment (start 5.55001 62.7104) (end 5.55001 64.3696) (width 0.25) (layer B.Cu) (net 8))
 (segment (start -13.94498 65.21502) (end -16 63.16) (width 0.25) (layer B.Cu) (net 8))
 (segment (start 4.70459 65.21502) (end -13.94498 65.21502) (width 0.25) (layer B.Cu) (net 8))
 (segment (start -12.596401 61.483599) (end -13.46 60.62) (width 0.25) (layer B.Cu) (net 6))
 (segment (start -11.76501 62.31499) (end -12.596401 61.483599) (width 0.25) (layer B.Cu) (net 6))
 (segment (start 2.49 62.64) (end 2.16499 62.31499) (width 0.25) (layer B.Cu) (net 6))
 (segment (start 2.16499 62.31499) (end -11.76501 62.31499) (width 0.25) (layer B.Cu) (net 6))
 (segment (start 2.49 63.54) (end 2.49 62.64) (width 0.25) (layer B.Cu) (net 6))
 (segment (start -15.136401 58.975531) (end -15.136401 59.756401) (width 0.25) (layer B.Cu) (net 9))
 (segment (start -15.136401 59.756401) (end -16 60.62) (width 0.25) (layer B.Cu) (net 9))
 (segment (start -14.811399 57.585502) (end -14.811399 58.650529) (width 0.25) (layer B.Cu) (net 9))
 (segment (start -14.811399 58.650529) (end -15.136401 58.975531) (width 0.25) (layer B.Cu) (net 9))
 (segment (start -14.117296 56.891399) (end -14.811399 57.585502) (width 0.25) (layer B.Cu) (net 9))
 (segment (start 0.301399 56.891399) (end -14.117296 56.891399) (width 0.25) (layer B.Cu) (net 9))
 (segment (start 3.51 60.1) (end 0.301399 56.891399) (width 0.25) (layer B.Cu) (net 9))
 (segment (start 3.51 61) (end 3.51 60.1) (width 0.25) (layer B.Cu) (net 9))
 (segment (start -14.323599 58.943599) (end -13.46 58.08) (width 0.25) (layer B.Cu) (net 10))
 (segment (start -14.648601 59.268601) (end -14.323599 58.943599) (width 0.25) (layer B.Cu) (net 10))
 (segment (start -13.61412 64.76501) (end -14.648601 63.730529) (width 0.25) (layer B.Cu) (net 10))
 (segment (start 4.19999 64.76501) (end -13.61412 64.76501) (width 0.25) (layer B.Cu) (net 10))
 (segment (start 4.525 64.44) (end 4.19999 64.76501) (width 0.25) (layer B.Cu) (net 10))
 (segment (start -14.648601 63.730529) (end -14.648601 59.268601) (width 0.25) (layer B.Cu) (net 10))
 (segment (start 4.525 63.54) (end 4.525 64.44) (width 0.25) (layer B.Cu) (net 10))
 (segment (start -13.08 63.54) (end -13.46 63.16) (width 0.25) (layer B.Cu) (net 7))
 (segment (start 0.46 63.54) (end -13.08 63.54) (width 0.25) (layer B.Cu) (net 7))
 (segment (start 16.150001 59.310001) (end 17 60.16) (width 0.25) (layer B.Cu) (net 2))
 (segment (start 13.243599 56.403599) (end 16.150001 59.310001) (width 0.25) (layer B.Cu) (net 2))
 (segment (start -12.596401 56.403599) (end 13.243599 56.403599) (width 0.25) (layer B.Cu) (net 2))
 (segment (start -13.46 55.54) (end -12.596401 56.403599) (width 0.25) (layer B.Cu) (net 2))
 (segment (start 16.150001 56.770001) (end 17 57.62) (width 0.25) (layer B.Cu) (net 3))
 (segment (start -5.116857 55.953589) (end 15.333589 55.953589) (width 0.25) (layer B.Cu) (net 3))
 (segment (start 15.333589 55.953589) (end 16.150001 56.770001) (width 0.25) (layer B.Cu) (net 3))
 (segment (start -6.719047 54.351399) (end -5.116857 55.953589) (width 0.25) (layer B.Cu) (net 3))
 (segment (start -14.811399 54.351399) (end -6.719047 54.351399) (width 0.25) (layer B.Cu) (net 3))
 (segment (start -16 55.54) (end -14.811399 54.351399) (width 0.25) (layer B.Cu) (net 3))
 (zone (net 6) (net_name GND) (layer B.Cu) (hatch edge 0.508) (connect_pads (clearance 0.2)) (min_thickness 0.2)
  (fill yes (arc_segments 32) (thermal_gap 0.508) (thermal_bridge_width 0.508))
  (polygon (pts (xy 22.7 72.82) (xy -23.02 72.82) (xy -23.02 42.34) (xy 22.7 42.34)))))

